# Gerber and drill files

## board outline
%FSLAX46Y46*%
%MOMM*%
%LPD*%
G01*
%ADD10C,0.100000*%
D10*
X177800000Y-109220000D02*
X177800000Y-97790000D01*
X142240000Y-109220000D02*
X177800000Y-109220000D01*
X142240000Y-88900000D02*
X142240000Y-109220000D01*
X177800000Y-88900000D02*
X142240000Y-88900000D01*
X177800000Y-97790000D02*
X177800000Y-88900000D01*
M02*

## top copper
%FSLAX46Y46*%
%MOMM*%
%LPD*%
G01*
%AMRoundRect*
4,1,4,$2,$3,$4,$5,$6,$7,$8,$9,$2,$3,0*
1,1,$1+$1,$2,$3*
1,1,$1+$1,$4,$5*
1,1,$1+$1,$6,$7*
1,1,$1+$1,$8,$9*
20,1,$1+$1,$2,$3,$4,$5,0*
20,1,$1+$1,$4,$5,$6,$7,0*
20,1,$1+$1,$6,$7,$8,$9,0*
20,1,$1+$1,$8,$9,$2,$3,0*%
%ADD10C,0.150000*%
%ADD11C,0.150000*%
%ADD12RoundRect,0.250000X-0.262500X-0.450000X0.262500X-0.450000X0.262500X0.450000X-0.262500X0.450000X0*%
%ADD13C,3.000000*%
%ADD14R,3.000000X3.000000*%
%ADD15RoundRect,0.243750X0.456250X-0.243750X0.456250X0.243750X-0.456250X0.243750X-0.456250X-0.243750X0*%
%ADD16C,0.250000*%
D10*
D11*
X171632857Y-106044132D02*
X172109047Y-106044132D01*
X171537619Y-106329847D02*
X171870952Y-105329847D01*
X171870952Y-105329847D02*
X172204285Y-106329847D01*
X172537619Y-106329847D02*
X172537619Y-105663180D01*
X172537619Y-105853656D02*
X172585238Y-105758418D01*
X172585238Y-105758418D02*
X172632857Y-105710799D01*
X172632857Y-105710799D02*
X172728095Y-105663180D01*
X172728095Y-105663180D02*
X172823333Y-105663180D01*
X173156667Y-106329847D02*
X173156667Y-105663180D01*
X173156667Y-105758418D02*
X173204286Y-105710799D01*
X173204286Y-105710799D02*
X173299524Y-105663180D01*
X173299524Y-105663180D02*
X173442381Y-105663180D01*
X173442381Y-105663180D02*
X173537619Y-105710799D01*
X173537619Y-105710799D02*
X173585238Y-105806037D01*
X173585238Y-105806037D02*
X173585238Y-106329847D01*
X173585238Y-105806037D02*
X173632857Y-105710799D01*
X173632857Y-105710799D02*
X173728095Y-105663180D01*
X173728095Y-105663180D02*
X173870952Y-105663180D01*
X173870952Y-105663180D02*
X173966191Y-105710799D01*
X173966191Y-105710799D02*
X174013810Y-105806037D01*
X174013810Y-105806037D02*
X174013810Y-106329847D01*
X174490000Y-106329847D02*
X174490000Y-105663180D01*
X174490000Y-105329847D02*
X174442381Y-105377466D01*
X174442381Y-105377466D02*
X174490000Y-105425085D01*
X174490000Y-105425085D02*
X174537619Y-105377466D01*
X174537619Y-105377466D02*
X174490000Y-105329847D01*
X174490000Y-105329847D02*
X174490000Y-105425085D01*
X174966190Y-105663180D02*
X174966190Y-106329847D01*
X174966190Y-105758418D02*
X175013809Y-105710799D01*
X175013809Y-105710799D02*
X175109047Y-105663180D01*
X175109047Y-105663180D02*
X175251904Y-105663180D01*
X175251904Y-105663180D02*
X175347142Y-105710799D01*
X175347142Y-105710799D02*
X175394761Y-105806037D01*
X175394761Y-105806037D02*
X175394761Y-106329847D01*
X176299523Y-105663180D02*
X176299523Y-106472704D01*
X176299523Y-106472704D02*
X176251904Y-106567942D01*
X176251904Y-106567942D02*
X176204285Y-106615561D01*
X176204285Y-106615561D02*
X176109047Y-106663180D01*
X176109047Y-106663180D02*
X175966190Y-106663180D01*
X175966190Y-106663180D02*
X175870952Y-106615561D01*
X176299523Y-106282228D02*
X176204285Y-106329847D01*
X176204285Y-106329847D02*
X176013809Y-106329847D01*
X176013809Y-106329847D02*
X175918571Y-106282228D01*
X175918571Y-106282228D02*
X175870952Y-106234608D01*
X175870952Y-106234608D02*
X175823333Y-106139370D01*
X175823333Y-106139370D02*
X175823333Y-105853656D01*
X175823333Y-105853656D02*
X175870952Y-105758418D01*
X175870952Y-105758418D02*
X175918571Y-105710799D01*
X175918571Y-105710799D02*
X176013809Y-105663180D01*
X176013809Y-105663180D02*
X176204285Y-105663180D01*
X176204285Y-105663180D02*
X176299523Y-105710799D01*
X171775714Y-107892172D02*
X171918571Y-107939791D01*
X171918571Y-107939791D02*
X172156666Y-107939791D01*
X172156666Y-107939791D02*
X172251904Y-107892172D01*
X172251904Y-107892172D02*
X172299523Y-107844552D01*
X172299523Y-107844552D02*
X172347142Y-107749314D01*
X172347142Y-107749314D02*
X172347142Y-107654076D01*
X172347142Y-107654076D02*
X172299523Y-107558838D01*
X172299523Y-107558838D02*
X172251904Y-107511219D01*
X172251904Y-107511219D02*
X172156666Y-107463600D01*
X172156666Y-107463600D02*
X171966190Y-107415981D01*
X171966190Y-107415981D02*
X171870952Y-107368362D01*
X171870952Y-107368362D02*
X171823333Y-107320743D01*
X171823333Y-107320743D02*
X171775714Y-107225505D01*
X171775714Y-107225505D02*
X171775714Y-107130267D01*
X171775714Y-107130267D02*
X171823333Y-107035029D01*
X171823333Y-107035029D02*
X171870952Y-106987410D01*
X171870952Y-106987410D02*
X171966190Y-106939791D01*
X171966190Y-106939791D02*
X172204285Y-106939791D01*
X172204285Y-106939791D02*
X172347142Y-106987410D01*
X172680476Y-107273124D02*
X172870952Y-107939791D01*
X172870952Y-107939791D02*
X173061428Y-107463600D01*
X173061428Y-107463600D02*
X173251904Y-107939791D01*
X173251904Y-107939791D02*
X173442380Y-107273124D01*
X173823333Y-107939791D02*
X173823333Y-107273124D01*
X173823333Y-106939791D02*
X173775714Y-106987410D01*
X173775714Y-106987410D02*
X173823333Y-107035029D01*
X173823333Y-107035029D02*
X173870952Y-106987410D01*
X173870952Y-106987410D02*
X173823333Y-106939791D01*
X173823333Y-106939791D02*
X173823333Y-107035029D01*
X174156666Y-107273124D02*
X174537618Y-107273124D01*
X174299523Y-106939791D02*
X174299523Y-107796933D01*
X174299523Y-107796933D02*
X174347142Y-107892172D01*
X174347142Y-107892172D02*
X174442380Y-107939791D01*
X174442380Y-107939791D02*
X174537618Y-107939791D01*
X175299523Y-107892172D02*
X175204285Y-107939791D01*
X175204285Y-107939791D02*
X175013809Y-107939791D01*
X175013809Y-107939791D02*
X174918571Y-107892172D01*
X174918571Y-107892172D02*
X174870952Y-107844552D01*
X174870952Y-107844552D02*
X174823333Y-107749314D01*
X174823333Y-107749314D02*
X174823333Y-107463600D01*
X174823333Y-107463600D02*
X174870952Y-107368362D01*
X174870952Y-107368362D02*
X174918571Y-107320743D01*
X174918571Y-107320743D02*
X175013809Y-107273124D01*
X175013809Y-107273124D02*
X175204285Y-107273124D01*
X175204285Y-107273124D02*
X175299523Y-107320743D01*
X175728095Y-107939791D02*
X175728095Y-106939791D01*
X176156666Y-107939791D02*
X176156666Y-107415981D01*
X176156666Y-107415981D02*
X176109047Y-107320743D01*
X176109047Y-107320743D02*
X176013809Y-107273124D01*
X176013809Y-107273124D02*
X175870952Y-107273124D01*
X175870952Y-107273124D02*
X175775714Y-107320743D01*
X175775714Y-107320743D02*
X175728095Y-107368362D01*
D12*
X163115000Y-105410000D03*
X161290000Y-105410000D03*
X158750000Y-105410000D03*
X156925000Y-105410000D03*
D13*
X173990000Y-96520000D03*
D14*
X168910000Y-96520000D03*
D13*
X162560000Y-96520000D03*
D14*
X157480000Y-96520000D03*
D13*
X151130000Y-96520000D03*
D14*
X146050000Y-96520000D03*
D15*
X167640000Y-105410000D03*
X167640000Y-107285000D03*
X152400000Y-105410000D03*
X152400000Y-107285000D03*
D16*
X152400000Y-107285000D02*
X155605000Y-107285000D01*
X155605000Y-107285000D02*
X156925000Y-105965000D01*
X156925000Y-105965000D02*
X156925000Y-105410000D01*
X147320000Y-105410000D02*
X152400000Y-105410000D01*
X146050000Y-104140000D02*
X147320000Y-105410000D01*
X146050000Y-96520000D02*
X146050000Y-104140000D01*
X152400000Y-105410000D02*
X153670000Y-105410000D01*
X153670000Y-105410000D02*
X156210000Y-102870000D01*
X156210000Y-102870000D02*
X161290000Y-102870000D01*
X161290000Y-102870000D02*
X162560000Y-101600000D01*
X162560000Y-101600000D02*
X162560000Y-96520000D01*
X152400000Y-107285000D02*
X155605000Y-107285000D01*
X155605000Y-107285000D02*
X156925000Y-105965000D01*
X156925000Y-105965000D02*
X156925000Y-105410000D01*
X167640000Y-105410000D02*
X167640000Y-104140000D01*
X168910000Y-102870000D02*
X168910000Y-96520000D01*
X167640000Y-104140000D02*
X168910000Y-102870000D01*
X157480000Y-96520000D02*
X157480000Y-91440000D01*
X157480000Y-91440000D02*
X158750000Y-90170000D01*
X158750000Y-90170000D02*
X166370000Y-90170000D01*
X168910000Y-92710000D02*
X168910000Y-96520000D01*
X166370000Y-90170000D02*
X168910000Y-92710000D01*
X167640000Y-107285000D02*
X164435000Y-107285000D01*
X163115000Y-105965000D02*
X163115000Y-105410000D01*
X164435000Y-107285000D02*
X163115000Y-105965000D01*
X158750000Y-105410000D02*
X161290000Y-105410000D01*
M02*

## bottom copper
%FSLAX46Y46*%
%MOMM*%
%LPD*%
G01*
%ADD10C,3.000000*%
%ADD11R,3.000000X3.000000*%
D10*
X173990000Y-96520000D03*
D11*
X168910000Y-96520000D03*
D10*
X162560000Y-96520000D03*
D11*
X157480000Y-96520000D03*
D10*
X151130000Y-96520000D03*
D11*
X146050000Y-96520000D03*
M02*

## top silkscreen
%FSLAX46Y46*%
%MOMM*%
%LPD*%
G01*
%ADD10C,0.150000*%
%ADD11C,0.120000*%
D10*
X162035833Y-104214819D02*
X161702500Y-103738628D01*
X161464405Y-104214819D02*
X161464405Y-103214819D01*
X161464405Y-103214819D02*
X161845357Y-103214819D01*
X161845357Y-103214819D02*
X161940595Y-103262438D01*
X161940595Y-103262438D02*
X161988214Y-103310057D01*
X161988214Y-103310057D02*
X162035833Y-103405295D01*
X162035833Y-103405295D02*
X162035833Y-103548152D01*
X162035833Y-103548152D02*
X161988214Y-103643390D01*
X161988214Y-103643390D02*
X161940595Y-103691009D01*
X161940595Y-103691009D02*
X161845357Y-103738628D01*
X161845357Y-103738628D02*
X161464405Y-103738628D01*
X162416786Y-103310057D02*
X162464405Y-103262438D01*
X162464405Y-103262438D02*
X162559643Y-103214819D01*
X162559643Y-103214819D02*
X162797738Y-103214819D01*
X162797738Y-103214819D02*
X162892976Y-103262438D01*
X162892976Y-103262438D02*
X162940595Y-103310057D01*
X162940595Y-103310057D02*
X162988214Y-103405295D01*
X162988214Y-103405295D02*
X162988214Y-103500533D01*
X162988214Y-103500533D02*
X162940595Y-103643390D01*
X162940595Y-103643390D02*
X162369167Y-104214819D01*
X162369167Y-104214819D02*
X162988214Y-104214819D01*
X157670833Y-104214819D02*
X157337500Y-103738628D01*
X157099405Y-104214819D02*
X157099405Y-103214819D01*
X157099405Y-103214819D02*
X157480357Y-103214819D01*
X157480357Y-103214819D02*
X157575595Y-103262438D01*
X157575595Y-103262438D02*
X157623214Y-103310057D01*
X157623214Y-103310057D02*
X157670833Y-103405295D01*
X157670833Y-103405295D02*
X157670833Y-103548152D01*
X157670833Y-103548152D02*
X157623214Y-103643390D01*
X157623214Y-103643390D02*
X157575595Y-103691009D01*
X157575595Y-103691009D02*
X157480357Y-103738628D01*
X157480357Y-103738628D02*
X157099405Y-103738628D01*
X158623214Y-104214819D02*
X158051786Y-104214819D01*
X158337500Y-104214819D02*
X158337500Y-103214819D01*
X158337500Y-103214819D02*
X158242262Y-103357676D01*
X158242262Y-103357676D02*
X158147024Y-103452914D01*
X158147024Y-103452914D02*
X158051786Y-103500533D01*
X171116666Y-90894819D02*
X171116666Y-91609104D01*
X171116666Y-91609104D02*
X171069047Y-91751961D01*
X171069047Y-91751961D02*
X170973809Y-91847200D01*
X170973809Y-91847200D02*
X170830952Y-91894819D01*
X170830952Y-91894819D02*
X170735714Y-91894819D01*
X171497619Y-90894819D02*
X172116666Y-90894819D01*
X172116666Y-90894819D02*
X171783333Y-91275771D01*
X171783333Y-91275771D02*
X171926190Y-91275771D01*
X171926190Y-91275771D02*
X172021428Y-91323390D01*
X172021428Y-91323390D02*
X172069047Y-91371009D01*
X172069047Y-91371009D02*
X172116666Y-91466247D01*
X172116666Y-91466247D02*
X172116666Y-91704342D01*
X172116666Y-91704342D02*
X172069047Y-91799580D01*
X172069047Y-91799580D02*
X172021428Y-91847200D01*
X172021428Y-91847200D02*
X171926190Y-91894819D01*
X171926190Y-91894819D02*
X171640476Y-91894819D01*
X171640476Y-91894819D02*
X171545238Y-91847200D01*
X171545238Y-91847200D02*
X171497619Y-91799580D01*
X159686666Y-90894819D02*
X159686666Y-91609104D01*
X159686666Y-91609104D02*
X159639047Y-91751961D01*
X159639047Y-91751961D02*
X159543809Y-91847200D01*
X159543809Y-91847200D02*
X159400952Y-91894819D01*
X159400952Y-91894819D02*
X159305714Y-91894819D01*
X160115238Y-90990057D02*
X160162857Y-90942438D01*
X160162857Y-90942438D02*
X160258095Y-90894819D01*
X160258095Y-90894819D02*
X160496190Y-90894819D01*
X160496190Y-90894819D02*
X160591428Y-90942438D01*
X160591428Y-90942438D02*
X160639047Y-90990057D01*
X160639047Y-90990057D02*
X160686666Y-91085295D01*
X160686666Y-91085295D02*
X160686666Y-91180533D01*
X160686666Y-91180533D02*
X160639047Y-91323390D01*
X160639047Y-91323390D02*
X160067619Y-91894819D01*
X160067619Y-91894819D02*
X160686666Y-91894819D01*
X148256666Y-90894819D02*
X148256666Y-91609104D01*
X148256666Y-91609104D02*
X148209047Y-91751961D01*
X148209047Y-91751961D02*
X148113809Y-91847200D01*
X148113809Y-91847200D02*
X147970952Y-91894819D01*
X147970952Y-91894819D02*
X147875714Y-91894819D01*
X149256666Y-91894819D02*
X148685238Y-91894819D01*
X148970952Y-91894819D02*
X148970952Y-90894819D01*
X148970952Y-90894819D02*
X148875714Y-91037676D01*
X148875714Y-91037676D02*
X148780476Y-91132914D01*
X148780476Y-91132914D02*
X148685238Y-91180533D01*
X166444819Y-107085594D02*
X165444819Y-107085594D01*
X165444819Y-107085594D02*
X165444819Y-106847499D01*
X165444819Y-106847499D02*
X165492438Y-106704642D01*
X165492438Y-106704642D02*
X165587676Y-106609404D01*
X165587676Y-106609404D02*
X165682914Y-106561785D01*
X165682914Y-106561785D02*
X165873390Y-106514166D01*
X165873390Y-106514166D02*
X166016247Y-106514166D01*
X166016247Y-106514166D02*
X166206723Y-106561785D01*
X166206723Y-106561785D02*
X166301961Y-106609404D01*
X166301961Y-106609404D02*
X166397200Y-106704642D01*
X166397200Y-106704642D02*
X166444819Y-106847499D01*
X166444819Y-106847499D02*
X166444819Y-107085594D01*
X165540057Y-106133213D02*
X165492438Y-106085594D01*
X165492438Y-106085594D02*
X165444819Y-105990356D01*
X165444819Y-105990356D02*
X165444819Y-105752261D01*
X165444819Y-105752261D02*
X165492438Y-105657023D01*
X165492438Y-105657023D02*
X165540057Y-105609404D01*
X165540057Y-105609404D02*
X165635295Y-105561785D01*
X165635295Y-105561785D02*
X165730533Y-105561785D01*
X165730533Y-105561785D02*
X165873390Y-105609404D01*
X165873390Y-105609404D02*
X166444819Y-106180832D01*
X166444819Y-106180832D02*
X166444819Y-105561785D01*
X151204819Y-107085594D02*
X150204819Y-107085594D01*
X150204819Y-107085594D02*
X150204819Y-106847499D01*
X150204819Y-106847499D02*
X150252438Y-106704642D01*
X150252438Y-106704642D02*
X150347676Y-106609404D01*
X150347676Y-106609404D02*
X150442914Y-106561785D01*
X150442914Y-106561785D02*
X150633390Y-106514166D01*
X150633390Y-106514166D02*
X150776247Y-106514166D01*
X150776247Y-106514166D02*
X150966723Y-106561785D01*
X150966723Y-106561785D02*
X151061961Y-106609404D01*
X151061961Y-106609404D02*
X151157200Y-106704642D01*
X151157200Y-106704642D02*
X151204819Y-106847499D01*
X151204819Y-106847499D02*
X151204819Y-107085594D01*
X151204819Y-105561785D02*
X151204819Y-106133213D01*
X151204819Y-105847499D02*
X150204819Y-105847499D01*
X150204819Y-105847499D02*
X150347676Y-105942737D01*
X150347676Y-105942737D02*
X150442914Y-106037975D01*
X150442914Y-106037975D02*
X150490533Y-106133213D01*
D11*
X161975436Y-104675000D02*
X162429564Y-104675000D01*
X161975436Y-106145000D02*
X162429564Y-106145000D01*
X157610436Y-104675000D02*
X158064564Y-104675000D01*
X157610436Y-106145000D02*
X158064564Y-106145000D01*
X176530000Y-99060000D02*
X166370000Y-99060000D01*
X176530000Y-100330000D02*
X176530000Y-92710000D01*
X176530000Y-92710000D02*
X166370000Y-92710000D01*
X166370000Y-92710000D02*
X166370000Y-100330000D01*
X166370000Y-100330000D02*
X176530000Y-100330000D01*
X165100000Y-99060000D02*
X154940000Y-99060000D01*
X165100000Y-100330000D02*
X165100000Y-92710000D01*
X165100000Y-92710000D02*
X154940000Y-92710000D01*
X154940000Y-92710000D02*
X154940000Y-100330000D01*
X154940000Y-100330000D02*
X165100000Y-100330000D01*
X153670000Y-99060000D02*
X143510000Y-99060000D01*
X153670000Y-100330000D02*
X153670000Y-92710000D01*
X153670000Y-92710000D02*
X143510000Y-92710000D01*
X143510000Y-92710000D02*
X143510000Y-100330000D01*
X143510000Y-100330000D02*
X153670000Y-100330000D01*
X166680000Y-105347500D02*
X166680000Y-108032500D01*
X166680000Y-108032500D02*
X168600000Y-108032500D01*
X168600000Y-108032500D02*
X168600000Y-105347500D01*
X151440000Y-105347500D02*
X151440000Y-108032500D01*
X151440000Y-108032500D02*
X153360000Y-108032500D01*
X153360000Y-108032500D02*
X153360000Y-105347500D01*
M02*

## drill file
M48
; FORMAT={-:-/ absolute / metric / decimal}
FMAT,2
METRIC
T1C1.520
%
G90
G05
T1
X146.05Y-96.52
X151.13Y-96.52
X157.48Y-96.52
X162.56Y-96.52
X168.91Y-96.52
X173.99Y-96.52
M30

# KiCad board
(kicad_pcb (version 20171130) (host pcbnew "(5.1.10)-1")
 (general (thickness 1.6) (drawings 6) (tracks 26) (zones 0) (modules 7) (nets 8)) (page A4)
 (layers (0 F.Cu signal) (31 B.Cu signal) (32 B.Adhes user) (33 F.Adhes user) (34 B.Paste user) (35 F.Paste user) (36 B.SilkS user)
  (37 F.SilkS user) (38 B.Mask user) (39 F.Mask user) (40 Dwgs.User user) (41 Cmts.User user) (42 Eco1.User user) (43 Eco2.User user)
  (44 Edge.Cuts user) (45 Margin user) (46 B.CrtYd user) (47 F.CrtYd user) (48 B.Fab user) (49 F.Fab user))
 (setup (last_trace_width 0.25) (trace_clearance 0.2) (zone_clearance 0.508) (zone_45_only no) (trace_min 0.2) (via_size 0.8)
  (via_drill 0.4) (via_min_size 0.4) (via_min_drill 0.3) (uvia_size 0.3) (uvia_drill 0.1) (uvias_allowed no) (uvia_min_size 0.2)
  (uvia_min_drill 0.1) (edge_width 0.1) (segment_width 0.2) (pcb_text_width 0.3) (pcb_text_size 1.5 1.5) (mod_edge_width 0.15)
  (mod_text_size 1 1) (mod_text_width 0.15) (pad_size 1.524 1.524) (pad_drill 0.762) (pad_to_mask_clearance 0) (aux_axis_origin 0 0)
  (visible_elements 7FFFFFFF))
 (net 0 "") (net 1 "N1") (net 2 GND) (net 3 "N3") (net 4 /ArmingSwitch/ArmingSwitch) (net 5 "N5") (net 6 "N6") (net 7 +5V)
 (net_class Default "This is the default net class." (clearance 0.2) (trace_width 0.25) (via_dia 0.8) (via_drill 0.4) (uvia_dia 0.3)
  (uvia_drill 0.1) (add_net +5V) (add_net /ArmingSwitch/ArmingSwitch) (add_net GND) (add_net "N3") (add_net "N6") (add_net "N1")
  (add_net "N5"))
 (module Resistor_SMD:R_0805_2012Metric (layer F.Cu) (at 162.2025 105.41)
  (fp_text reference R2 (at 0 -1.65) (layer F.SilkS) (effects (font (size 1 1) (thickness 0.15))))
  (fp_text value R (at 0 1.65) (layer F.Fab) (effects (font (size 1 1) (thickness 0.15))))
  (fp_line (start -0.227064 -0.735) (end 0.227064 -0.735) (layer F.SilkS) (width 0.12))
  (fp_line (start -0.227064 0.735) (end 0.227064 0.735) (layer F.SilkS) (width 0.12))
  (pad 2 smd roundrect (at 0.9125 0) (size 1.025 1.4) (layers F.Cu F.Paste F.Mask) (roundrect_rratio 0.243902) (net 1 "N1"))
  (pad 1 smd roundrect (at -0.9125 0) (size 1.025 1.4) (layers F.Cu F.Paste F.Mask) (roundrect_rratio 0.243902) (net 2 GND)))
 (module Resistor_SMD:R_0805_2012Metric (layer F.Cu) (at 157.8375 105.41)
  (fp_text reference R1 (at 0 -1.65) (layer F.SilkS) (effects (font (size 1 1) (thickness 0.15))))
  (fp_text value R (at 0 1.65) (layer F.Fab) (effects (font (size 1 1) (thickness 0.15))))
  (fp_line (start -0.227064 -0.735) (end 0.227064 -0.735) (layer F.SilkS) (width 0.12))
  (fp_line (start -0.227064 0.735) (end 0.227064 0.735) (layer F.SilkS) (width 0.12))
  (pad 2 smd roundrect (at 0.9125 0) (size 1.025 1.4) (layers F.Cu F.Paste F.Mask) (roundrect_rratio 0.243902) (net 2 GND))
  (pad 1 smd roundrect (at -0.9125 0) (size 1.025 1.4) (layers F.Cu F.Paste F.Mask) (roundrect_rratio 0.243902) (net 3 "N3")))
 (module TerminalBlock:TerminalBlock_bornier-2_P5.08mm (layer F.Cu) (at 168.91 96.52)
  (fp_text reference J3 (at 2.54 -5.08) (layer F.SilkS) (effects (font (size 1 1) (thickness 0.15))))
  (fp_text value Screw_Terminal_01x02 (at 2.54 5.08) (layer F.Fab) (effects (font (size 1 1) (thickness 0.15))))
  (fp_line (start 7.62 2.54) (end -2.54 2.54) (layer F.SilkS) (width 0.12))
  (fp_line (start 7.62 3.81) (end 7.62 -3.81) (layer F.SilkS) (width 0.12))
  (fp_line (start 7.62 -3.81) (end -2.54 -3.81) (layer F.SilkS) (width 0.12))
  (fp_line (start -2.54 -3.81) (end -2.54 3.81) (layer F.SilkS) (width 0.12))
  (fp_line (start -2.54 3.81) (end 7.62 3.81) (layer F.SilkS) (width 0.12))
  (pad 2 thru_hole circle (at 5.08 0) (size 3 3) (drill 1.52) (layers *.Cu *.Mask) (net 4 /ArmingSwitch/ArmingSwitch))
  (pad 1 thru_hole rect (at 0 0) (size 3 3) (drill 1.52) (layers *.Cu *.Mask) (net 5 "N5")))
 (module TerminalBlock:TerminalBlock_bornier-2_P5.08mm (layer F.Cu) (at 157.48 96.52)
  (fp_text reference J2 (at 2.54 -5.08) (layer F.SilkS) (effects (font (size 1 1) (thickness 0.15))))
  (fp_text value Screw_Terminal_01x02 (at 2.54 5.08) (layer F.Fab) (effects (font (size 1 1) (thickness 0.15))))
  (fp_line (start 7.62 2.54) (end -2.54 2.54) (layer F.SilkS) (width 0.12))
  (fp_line (start 7.62 3.81) (end 7.62 -3.81) (layer F.SilkS) (width 0.12))
  (fp_line (start 7.62 -3.81) (end -2.54 -3.81) (layer F.SilkS) (width 0.12))
  (fp_line (start -2.54 -3.81) (end -2.54 3.81) (layer F.SilkS) (width 0.12))
  (fp_line (start -2.54 3.81) (end 7.62 3.81) (layer F.SilkS) (width 0.12))
  (pad 2 thru_hole circle (at 5.08 0) (size 3 3) (drill 1.52) (layers *.Cu *.Mask) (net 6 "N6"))
  (pad 1 thru_hole rect (at 0 0) (size 3 3) (drill 1.52) (layers *.Cu *.Mask) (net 5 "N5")))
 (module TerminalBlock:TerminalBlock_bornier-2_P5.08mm (layer F.Cu) (at 146.05 96.52)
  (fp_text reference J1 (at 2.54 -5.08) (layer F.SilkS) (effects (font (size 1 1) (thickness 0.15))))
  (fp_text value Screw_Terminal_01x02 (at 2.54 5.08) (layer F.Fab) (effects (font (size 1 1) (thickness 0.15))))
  (fp_line (start 7.62 2.54) (end -2.54 2.54) (layer F.SilkS) (width 0.12))
  (fp_line (start 7.62 3.81) (end 7.62 -3.81) (layer F.SilkS) (width 0.12))
  (fp_line (start 7.62 -3.81) (end -2.54 -3.81) (layer F.SilkS) (width 0.12))
  (fp_line (start -2.54 -3.81) (end -2.54 3.81) (layer F.SilkS) (width 0.12))
  (fp_line (start -2.54 3.81) (end 7.62 3.81) (layer F.SilkS) (width 0.12))
  (pad 2 thru_hole circle (at 5.08 0) (size 3 3) (drill 1.52) (layers *.Cu *.Mask) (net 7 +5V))
  (pad 1 thru_hole rect (at 0 0) (size 3 3) (drill 1.52) (layers *.Cu *.Mask) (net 6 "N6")))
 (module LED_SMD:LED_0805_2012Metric (layer F.Cu) (at 167.64 106.3475 90)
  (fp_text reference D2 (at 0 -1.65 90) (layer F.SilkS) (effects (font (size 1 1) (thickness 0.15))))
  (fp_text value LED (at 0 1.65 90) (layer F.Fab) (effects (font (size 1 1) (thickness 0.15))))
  (fp_line (start 1 -0.96) (end -1.685 -0.96) (layer F.SilkS) (width 0.12))
  (fp_line (start -1.685 -0.96) (end -1.685 0.96) (layer F.SilkS) (width 0.12))
  (fp_line (start -1.685 0.96) (end 1 0.96) (layer F.SilkS) (width 0.12))
  (pad 2 smd roundrect (at 0.9375 0 90) (size 0.975 1.4) (layers F.Cu F.Paste F.Mask) (roundrect_rratio 0.25) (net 5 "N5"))
  (pad 1 smd roundrect (at -0.9375 0 90) (size 0.975 1.4) (layers F.Cu F.Paste F.Mask) (roundrect_rratio 0.25) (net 1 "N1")))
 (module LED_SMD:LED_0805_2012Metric (layer F.Cu) (at 152.4 106.3475 90)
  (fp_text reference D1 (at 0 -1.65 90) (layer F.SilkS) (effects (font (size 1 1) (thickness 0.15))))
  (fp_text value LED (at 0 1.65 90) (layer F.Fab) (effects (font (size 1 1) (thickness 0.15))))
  (fp_line (start 1 -0.96) (end -1.685 -0.96) (layer F.SilkS) (width 0.12))
  (fp_line (start -1.685 -0.96) (end -1.685 0.96) (layer F.SilkS) (width 0.12))
  (fp_line (start -1.685 0.96) (end 1 0.96) (layer F.SilkS) (width 0.12))
  (pad 2 smd roundrect (at 0.9375 0 90) (size 0.975 1.4) (layers F.Cu F.Paste F.Mask) (roundrect_rratio 0.25) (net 6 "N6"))
  (pad 1 smd roundrect (at -0.9375 0 90) (size 0.975 1.4) (layers F.Cu F.Paste F.Mask) (roundrect_rratio 0.25) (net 3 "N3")))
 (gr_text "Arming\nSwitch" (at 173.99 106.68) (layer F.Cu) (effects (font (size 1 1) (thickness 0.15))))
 (gr_line (start 177.8 109.22) (end 177.8 97.79) (layer Edge.Cuts) (width 0.1))
 (gr_line (start 142.24 109.22) (end 177.8 109.22) (layer Edge.Cuts) (width 0.1))
 (gr_line (start 142.24 88.9) (end 142.24 109.22) (layer Edge.Cuts) (width 0.1))
 (gr_line (start 177.8 88.9) (end 142.24 88.9) (layer Edge.Cuts) (width 0.1))
 (gr_line (start 177.8 97.79) (end 177.8 88.9) (layer Edge.Cuts) (width 0.1))
 (segment (start 152.4 107.285) (end 155.605 107.285) (width 0.25) (layer F.Cu) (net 3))
 (segment (start 155.605 107.285) (end 156.925 105.965) (width 0.25) (layer F.Cu) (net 3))
 (segment (start 156.925 105.965) (end 156.925 105.41) (width 0.25) (layer F.Cu) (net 3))
 (segment (start 147.32 105.41) (end 152.4 105.41) (width 0.25) (layer F.Cu) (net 6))
 (segment (start 146.05 104.14) (end 147.32 105.41) (width 0.25) (layer F.Cu) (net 6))
 (segment (start 146.05 96.52) (end 146.05 104.14) (width 0.25) (layer F.Cu) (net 6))
 (segment (start 152.4 105.41) (end 153.67 105.41) (width 0.25) (layer F.Cu) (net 6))
 (segment (start 153.67 105.41) (end 156.21 102.87) (width 0.25) (layer F.Cu) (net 6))
 (segment (start 156.21 102.87) (end 161.29 102.87) (width 0.25) (layer F.Cu) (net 6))
 (segment (start 161.29 102.87) (end 162.56 101.6) (width 0.25) (layer F.Cu) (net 6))
 (segment (start 162.56 101.6) (end 162.56 96.52) (width 0.25) (layer F.Cu) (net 6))
 (segment (start 152.4 107.285) (end 155.605 107.285) (width 0.25) (layer F.Cu) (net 3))
 (segment (start 155.605 107.285) (end 156.925 105.965) (width 0.25) (layer F.Cu) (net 3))
 (segment (start 156.925 105.965) (end 156.925 105.41) (width 0.25) (layer F.Cu) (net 3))
 (segment (start 167.64 105.41) (end 167.64 104.14) (width 0.25) (layer F.Cu) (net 5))
 (segment (start 168.91 102.87) (end 168.91 96.52) (width 0.25) (layer F.Cu) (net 5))
 (segment (start 167.64 104.14) (end 168.91 102.87) (width 0.25) (layer F.Cu) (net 5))
 (segment (start 157.48 96.52) (end 157.48 91.44) (width 0.25) (layer F.Cu) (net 5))
 (segment (start 157.48 91.44) (end 158.75 90.17) (width 0.25) (layer F.Cu) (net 5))
 (segment (start 158.75 90.17) (end 166.37 90.17) (width 0.25) (layer F.Cu) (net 5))
 (segment (start 168.91 92.71) (end 168.91 96.52) (width 0.25) (layer F.Cu) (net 5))
 (segment (start 166.37 90.17) (end 168.91 92.71) (width 0.25) (layer F.Cu) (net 5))
 (segment (start 167.64 107.285) (end 164.435 107.285) (width 0.25) (layer F.Cu) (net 1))
 (segment (start 163.115 105.965) (end 163.115 105.41) (width 0.25) (layer F.Cu) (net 1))
 (segment (start 164.435 107.285) (end 163.115 105.965) (width 0.25) (layer F.Cu) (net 1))
 (segment (start 158.75 105.41) (end 161.29 105.41) (width 0.25) (layer F.Cu) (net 2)))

